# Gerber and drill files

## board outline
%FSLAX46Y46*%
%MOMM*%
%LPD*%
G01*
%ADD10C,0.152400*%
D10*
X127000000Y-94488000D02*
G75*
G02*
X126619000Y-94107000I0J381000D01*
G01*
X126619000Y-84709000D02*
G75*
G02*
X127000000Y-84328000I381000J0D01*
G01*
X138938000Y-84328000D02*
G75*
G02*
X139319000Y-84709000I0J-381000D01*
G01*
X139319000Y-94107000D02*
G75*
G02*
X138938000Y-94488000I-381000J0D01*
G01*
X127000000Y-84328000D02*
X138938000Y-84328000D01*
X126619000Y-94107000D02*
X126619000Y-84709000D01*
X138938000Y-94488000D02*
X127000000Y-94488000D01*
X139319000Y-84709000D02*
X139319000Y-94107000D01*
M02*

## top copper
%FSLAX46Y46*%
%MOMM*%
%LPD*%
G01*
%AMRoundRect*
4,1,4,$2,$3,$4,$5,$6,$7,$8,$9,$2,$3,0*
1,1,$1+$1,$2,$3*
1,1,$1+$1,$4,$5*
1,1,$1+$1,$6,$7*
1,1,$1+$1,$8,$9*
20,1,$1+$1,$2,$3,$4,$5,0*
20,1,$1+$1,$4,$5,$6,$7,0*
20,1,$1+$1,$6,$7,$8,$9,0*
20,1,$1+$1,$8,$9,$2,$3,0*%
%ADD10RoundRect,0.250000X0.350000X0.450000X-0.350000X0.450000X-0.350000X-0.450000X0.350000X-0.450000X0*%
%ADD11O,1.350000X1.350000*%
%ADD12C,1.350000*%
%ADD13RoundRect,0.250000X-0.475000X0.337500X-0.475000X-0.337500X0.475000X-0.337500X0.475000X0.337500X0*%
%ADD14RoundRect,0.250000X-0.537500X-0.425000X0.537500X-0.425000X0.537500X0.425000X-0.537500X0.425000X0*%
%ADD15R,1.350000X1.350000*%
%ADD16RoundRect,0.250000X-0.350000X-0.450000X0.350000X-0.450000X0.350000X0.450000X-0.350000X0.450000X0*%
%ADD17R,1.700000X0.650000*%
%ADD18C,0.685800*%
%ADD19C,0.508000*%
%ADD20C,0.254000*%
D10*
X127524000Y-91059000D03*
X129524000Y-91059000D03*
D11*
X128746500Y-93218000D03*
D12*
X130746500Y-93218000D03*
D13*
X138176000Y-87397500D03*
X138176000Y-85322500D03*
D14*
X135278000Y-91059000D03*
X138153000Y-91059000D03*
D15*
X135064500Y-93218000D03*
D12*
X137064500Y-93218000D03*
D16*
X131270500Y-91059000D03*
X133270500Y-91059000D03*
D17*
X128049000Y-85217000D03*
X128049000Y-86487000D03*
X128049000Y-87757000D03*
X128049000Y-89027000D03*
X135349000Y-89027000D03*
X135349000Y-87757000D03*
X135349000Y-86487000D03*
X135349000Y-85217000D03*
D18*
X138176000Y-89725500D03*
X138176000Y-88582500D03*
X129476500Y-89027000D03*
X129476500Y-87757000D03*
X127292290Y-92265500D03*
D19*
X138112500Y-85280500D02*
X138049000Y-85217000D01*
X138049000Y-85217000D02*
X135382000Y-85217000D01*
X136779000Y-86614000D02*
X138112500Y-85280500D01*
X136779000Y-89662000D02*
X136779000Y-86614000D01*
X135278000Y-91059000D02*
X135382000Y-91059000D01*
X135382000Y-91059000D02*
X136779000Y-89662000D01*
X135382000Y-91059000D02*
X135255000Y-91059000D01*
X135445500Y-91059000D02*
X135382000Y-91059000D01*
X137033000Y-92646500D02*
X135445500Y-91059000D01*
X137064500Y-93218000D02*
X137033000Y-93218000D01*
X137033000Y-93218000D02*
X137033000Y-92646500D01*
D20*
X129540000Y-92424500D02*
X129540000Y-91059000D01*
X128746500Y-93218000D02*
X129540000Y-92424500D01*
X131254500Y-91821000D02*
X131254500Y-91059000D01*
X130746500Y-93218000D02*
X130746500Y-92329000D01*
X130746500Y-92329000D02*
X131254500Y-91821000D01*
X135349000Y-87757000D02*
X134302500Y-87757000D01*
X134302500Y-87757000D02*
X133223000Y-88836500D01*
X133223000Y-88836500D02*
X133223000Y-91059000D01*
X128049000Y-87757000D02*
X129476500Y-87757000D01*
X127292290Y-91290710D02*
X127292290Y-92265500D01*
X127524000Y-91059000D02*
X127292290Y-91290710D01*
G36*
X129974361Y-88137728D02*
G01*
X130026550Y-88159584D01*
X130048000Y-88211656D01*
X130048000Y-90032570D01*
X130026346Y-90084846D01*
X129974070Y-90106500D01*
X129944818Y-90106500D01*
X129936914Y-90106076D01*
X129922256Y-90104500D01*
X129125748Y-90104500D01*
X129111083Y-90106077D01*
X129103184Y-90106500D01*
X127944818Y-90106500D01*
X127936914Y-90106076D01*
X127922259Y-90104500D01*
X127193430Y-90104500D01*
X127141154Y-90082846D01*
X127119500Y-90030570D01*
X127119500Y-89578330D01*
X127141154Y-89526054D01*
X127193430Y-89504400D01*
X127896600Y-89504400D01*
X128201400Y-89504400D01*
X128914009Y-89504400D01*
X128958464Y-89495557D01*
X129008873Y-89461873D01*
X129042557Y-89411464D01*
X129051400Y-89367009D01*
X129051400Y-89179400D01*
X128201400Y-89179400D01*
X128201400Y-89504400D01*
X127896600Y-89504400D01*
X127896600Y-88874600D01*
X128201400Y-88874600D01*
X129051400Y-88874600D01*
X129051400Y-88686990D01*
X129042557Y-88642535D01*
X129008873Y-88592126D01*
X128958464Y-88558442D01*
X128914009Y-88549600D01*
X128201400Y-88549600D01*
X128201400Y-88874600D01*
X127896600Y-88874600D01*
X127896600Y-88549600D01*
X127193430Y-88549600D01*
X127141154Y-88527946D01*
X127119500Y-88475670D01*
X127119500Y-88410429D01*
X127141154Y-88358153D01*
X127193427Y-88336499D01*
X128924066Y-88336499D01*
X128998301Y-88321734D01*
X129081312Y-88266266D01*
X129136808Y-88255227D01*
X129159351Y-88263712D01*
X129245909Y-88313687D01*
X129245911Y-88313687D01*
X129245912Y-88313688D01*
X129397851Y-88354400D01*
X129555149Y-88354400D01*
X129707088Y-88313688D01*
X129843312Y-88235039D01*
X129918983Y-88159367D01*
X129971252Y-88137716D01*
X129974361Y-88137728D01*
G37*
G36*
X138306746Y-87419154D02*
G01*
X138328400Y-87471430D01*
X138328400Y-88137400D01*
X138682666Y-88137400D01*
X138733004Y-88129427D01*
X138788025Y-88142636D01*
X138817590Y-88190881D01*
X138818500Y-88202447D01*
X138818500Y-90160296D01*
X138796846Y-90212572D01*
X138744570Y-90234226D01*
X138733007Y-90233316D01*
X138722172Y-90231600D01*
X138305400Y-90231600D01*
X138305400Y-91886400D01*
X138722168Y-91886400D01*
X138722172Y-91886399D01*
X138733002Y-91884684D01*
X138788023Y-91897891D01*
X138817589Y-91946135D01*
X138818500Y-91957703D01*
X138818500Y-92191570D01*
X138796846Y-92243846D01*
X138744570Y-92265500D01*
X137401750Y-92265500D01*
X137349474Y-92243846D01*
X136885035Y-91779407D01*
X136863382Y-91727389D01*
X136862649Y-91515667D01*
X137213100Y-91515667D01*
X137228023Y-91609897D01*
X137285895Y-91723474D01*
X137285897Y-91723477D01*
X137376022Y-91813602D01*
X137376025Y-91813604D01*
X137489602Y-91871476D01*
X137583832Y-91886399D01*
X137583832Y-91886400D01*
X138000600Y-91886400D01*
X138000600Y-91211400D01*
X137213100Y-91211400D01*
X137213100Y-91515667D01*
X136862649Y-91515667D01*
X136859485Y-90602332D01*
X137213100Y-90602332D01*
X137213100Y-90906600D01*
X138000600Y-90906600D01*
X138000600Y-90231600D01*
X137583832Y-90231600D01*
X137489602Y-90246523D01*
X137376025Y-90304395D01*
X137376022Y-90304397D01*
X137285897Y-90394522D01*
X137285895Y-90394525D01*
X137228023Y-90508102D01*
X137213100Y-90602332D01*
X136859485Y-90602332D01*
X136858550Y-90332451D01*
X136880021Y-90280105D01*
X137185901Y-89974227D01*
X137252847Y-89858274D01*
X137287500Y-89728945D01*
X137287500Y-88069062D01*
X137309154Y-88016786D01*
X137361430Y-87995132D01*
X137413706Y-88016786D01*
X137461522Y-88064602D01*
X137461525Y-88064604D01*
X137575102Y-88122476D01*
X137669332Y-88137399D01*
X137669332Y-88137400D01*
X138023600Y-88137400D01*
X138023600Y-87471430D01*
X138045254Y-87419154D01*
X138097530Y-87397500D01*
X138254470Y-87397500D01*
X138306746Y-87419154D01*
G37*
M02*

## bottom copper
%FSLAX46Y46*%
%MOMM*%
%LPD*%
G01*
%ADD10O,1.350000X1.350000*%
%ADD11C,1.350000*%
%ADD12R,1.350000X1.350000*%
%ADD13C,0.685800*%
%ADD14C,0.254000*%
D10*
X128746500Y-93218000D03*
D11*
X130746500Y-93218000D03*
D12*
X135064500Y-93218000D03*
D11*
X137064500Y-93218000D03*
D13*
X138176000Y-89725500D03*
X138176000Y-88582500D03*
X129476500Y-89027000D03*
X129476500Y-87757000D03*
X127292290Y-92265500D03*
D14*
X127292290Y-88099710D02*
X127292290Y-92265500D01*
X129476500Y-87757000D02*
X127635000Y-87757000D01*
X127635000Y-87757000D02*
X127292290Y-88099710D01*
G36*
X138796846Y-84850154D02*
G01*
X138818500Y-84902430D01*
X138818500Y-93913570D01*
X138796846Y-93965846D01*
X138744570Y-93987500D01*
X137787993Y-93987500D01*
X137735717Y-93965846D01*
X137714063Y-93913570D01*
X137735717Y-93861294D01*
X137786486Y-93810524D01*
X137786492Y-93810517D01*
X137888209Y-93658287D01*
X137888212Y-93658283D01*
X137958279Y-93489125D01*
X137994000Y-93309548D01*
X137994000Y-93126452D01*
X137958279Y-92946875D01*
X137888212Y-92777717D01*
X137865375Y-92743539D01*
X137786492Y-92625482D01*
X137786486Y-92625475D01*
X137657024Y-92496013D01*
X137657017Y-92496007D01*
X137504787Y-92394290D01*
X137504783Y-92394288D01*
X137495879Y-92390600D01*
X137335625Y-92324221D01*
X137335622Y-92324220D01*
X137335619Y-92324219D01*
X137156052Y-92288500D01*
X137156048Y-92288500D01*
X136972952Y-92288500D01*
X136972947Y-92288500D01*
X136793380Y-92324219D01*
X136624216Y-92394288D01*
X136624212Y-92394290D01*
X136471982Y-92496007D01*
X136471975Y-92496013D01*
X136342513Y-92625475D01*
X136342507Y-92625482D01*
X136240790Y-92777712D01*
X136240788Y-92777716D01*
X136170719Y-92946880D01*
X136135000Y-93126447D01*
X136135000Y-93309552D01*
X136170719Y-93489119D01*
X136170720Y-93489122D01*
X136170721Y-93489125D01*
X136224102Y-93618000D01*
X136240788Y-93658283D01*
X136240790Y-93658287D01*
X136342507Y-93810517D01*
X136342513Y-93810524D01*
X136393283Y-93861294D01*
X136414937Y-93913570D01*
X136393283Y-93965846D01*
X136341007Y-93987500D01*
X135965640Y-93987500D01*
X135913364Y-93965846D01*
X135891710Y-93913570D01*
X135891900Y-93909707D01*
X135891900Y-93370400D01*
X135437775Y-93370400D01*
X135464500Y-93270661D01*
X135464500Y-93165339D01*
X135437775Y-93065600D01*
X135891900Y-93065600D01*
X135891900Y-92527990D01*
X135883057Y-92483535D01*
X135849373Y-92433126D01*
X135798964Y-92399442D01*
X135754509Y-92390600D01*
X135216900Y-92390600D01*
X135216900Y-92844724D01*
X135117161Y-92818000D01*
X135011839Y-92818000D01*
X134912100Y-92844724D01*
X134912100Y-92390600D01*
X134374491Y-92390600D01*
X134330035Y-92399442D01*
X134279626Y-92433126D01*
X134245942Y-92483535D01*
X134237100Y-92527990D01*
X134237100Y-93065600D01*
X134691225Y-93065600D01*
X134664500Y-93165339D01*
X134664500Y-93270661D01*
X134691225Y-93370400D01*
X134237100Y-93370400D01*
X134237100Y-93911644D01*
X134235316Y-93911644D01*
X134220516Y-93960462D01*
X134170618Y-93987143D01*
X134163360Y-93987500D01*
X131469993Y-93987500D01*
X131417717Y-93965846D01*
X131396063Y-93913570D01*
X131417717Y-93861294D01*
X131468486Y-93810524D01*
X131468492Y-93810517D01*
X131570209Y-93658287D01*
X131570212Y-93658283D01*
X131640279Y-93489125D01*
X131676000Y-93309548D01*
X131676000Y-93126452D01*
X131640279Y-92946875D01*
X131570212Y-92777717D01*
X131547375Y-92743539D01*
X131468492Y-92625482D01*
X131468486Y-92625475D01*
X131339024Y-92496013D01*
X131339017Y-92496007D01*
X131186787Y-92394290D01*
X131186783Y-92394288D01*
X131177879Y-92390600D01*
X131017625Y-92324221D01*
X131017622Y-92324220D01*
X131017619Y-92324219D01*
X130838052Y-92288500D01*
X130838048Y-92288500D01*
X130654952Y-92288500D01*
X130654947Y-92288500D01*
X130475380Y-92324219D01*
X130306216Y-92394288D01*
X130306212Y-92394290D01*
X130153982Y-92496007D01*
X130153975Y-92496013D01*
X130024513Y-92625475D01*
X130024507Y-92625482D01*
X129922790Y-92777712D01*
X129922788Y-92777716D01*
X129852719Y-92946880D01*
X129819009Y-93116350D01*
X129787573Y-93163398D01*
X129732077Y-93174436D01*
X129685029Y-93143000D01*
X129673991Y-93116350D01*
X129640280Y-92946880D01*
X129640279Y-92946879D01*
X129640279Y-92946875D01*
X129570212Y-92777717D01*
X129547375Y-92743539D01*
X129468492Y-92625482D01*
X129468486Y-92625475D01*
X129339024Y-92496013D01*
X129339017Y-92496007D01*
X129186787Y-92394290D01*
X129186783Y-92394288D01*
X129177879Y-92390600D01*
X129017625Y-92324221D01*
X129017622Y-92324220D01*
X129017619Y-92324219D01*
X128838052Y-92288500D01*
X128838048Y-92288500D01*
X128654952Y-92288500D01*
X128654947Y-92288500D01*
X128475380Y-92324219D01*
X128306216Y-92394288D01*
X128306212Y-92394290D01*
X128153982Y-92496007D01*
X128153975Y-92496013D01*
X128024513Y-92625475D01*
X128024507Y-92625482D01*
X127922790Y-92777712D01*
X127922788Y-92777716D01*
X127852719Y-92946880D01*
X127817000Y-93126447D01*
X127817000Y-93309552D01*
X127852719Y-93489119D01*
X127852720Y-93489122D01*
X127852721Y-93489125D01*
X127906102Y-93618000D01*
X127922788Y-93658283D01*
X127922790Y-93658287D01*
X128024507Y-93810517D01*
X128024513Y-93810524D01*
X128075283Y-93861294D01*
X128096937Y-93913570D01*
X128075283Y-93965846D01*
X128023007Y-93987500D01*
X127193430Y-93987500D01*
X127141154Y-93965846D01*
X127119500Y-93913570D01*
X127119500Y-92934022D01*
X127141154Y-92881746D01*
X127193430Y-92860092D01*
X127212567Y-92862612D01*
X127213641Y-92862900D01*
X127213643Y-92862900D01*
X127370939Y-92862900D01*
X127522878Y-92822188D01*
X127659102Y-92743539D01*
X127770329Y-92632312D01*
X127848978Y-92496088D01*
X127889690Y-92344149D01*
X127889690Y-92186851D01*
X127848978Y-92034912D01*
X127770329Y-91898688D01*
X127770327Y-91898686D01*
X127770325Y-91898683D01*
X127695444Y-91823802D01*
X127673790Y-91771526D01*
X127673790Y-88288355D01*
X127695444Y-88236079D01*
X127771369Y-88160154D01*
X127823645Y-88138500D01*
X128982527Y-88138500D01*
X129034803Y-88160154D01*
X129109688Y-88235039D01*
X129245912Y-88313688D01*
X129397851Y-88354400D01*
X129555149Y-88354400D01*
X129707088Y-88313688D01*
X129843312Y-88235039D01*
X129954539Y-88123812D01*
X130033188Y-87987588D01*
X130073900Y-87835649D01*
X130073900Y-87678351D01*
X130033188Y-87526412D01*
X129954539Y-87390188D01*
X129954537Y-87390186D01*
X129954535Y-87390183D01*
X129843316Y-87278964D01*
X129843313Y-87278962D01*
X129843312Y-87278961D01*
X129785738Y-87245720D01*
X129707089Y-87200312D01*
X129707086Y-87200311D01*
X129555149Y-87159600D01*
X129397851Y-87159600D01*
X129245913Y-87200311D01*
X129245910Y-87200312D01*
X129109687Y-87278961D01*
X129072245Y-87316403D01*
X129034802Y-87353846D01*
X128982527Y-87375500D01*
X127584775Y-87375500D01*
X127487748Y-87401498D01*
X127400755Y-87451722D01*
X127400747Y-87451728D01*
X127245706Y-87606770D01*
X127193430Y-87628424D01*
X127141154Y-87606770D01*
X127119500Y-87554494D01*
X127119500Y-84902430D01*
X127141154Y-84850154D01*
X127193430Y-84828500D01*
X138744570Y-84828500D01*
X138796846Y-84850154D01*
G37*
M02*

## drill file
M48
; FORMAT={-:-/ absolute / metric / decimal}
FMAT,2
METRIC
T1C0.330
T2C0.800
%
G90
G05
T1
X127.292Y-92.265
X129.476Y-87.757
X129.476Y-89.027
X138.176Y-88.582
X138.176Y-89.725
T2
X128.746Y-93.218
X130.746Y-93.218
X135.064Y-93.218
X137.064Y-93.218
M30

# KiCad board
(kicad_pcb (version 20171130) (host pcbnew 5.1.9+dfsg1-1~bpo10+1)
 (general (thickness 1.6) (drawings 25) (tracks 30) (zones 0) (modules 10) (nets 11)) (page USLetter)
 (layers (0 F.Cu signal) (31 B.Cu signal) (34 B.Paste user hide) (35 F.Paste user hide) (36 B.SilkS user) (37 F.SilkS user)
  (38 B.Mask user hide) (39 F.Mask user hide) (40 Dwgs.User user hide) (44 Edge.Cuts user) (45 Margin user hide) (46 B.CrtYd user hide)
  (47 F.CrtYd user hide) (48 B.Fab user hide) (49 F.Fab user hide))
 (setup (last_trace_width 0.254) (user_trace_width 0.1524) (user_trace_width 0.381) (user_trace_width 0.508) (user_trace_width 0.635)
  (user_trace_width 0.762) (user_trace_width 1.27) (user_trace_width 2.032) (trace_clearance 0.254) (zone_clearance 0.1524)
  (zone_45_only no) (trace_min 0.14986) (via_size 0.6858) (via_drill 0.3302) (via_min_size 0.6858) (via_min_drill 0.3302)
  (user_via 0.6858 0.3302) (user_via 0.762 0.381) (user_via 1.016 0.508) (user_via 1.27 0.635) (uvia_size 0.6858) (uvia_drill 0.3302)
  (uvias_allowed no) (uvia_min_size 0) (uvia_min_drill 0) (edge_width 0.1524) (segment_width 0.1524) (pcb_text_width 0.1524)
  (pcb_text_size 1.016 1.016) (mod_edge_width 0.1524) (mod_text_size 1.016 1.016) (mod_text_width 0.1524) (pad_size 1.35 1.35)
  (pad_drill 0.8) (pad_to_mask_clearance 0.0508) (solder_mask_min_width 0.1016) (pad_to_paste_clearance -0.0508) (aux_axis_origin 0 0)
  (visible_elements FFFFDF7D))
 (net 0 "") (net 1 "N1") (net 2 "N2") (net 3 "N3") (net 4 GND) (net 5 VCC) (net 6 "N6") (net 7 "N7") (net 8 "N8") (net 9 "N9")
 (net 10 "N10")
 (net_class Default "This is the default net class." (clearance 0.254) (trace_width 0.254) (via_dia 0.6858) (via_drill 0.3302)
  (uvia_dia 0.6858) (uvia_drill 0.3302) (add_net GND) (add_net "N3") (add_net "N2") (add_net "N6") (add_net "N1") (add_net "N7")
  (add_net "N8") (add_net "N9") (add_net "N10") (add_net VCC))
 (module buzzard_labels (layer B.Cu) (at 135.89 91.3765 180)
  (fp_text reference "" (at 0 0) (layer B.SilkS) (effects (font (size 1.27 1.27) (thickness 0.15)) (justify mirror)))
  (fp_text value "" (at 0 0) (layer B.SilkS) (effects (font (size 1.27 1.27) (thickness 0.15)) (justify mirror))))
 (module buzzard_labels (layer B.Cu) (at 129.667 91.3765 180)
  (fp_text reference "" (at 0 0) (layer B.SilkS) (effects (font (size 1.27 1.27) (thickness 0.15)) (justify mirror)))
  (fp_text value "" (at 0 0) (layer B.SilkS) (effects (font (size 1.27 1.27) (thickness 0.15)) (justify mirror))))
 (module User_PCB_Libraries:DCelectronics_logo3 (layer B.Cu) (at 133.223 86.36 180)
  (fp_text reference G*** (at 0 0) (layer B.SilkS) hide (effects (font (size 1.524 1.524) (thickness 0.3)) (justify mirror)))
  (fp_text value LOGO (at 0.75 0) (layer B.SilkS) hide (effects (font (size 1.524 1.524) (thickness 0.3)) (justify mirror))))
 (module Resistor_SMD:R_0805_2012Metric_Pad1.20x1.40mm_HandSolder (layer F.Cu) (at 128.524 91.059 180)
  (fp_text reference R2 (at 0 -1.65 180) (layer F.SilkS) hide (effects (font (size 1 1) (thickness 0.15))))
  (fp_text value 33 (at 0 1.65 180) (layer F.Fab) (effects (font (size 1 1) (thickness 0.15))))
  (pad 2 smd roundrect (at 1 0 180) (size 1.2 1.4) (layers F.Cu F.Paste F.Mask) (roundrect_rratio 0.208333) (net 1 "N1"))
  (pad 1 smd roundrect (at -1 0 180) (size 1.2 1.4) (layers F.Cu F.Paste F.Mask) (roundrect_rratio 0.208333) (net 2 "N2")))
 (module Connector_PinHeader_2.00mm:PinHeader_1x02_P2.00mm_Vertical (layer F.Cu) (at 130.7465 93.218 270)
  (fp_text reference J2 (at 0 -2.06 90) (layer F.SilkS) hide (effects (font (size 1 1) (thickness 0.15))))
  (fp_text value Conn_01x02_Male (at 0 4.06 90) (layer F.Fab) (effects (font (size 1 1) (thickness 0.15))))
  (pad 2 thru_hole oval (at 0 2 270) (size 1.35 1.35) (drill 0.8) (layers *.Cu *.Mask) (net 2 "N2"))
  (pad 1 thru_hole circle (at 0 0 270) (size 1.35 1.35) (drill 0.8) (layers *.Cu *.Mask) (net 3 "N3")))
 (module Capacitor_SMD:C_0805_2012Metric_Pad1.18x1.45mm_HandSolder (layer F.Cu) (at 138.176 86.36 270)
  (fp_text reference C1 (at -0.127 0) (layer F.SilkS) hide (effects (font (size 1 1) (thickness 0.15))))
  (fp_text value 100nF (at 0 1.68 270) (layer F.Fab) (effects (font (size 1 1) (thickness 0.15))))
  (pad 2 smd roundrect (at 1.0375 0 270) (size 1.175 1.45) (layers F.Cu F.Paste F.Mask) (roundrect_rratio 0.212766) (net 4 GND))
  (pad 1 smd roundrect (at -1.0375 0 270) (size 1.175 1.45) (layers F.Cu F.Paste F.Mask) (roundrect_rratio 0.212766) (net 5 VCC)))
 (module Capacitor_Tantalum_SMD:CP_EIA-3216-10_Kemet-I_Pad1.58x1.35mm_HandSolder (layer F.Cu) (at 136.7155 91.059)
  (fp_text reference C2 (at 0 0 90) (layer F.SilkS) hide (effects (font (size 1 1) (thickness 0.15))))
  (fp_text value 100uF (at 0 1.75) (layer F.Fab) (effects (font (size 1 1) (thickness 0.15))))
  (pad 1 smd roundrect (at -1.4375 0) (size 1.575 1.35) (layers F.Cu F.Paste F.Mask) (roundrect_rratio 0.185185) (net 5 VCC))
  (pad 2 smd roundrect (at 1.4375 0) (size 1.575 1.35) (layers F.Cu F.Paste F.Mask) (roundrect_rratio 0.185185) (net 4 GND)))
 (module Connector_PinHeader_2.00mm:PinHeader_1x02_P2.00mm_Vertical (layer F.Cu) (at 137.0645 93.218 270)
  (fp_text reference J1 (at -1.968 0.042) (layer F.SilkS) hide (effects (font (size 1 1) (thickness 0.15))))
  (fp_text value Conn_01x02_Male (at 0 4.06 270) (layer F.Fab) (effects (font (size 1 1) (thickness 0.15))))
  (pad 2 thru_hole rect (at 0 2 270) (size 1.35 1.35) (drill 0.8) (layers *.Cu *.Mask) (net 4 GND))
  (pad 1 thru_hole circle (at 0 0 270) (size 1.35 1.35) (drill 0.8) (layers *.Cu *.Mask) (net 5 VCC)))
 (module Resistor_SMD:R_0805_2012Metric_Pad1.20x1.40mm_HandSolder (layer F.Cu) (at 132.2705 91.059)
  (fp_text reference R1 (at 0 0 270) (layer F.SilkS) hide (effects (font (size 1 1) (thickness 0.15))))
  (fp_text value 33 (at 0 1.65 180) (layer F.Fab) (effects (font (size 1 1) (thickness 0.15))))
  (pad 1 smd roundrect (at -1 0) (size 1.2 1.4) (layers F.Cu F.Paste F.Mask) (roundrect_rratio 0.208333) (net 3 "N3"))
  (pad 2 smd roundrect (at 1 0) (size 1.2 1.4) (layers F.Cu F.Paste F.Mask) (roundrect_rratio 0.208333) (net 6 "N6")))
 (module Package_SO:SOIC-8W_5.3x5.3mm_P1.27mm (layer F.Cu) (at 131.699 87.122)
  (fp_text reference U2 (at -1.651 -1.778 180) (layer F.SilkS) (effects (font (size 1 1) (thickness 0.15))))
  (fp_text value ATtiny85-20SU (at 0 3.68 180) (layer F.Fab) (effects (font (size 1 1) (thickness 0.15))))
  (pad 1 smd rect (at -3.65 -1.905) (size 1.7 0.65) (layers F.Cu F.Paste F.Mask) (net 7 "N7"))
  (pad 2 smd rect (at -3.65 -0.635) (size 1.7 0.65) (layers F.Cu F.Paste F.Mask) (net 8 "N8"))
  (pad 3 smd rect (at -3.65 0.635) (size 1.7 0.65) (layers F.Cu F.Paste F.Mask) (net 1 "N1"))
  (pad 4 smd rect (at -3.65 1.905) (size 1.7 0.65) (layers F.Cu F.Paste F.Mask) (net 4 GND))
  (pad 5 smd rect (at 3.65 1.905) (size 1.7 0.65) (layers F.Cu F.Paste F.Mask) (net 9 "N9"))
  (pad 6 smd rect (at 3.65 0.635) (size 1.7 0.65) (layers F.Cu F.Paste F.Mask) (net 6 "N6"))
  (pad 7 smd rect (at 3.65 -0.635) (size 1.7 0.65) (layers F.Cu F.Paste F.Mask) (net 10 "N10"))
  (pad 8 smd rect (at 3.65 -1.905) (size 1.7 0.65) (layers F.Cu F.Paste F.Mask) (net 5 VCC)))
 (gr_arc (start 127 94.107) (end 126.619 94.107) (angle -90) (layer Edge.Cuts) (width 0.1524))
 (gr_arc (start 127 84.709) (end 127 84.328) (angle -90) (layer Edge.Cuts) (width 0.1524))
 (gr_arc (start 138.938 84.709) (end 139.319 84.709) (angle -90) (layer Edge.Cuts) (width 0.1524))
 (gr_arc (start 138.938 94.107) (end 138.938 94.488) (angle -90) (layer Edge.Cuts) (width 0.1524))
 (gr_line (start 127 84.328) (end 138.938 84.328) (layer Edge.Cuts) (width 0.1524))
 (gr_line (start 126.619 94.107) (end 126.619 84.709) (layer Edge.Cuts) (width 0.1524))
 (gr_line (start 138.938 94.488) (end 127 94.488) (layer Edge.Cuts) (width 0.1524))
 (gr_line (start 139.319 84.709) (end 139.319 94.107) (layer Edge.Cuts) (width 0.1524))
 (via (at 138.176 89.7255) (size 0.6858) (drill 0.3302) (layers F.Cu B.Cu) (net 4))
 (via (at 138.176 88.5825) (size 0.6858) (drill 0.3302) (layers F.Cu B.Cu) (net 4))
 (via (at 129.4765 89.027) (size 0.6858) (drill 0.3302) (layers F.Cu B.Cu) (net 4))
 (segment (start 138.1125 85.2805) (end 138.049 85.217) (width 0.508) (layer F.Cu) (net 5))
 (segment (start 138.049 85.217) (end 135.382 85.217) (width 0.508) (layer F.Cu) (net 5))
 (segment (start 136.779 86.614) (end 138.1125 85.2805) (width 0.508) (layer F.Cu) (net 5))
 (segment (start 136.779 89.662) (end 136.779 86.614) (width 0.508) (layer F.Cu) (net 5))
 (segment (start 135.278 91.059) (end 135.382 91.059) (width 0.508) (layer F.Cu) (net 5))
 (segment (start 135.382 91.059) (end 136.779 89.662) (width 0.508) (layer F.Cu) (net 5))
 (segment (start 135.382 91.059) (end 135.255 91.059) (width 0.508) (layer F.Cu) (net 5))
 (segment (start 135.4455 91.059) (end 135.382 91.059) (width 0.508) (layer F.Cu) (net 5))
 (segment (start 137.033 92.6465) (end 135.4455 91.059) (width 0.508) (layer F.Cu) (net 5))
 (segment (start 137.0645 93.218) (end 137.033 93.218) (width 0.508) (layer F.Cu) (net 5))
 (segment (start 137.033 93.218) (end 137.033 92.6465) (width 0.508) (layer F.Cu) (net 5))
 (segment (start 129.54 92.4245) (end 129.54 91.059) (width 0.254) (layer F.Cu) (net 2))
 (segment (start 128.7465 93.218) (end 129.54 92.4245) (width 0.254) (layer F.Cu) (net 2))
 (segment (start 131.2545 91.821) (end 131.2545 91.059) (width 0.254) (layer F.Cu) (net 3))
 (segment (start 130.7465 93.218) (end 130.7465 92.329) (width 0.254) (layer F.Cu) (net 3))
 (segment (start 130.7465 92.329) (end 131.2545 91.821) (width 0.254) (layer F.Cu) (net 3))
 (segment (start 135.349 87.757) (end 134.3025 87.757) (width 0.254) (layer F.Cu) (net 6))
 (segment (start 134.3025 87.757) (end 133.223 88.8365) (width 0.254) (layer F.Cu) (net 6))
 (segment (start 133.223 88.8365) (end 133.223 91.059) (width 0.254) (layer F.Cu) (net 6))
 (via (at 129.4765 87.757) (size 0.6858) (drill 0.3302) (layers F.Cu B.Cu) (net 1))
 (segment (start 128.049 87.757) (end 129.4765 87.757) (width 0.254) (layer F.Cu) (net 1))
 (via (at 127.29229 92.2655) (size 0.6858) (drill 0.3302) (layers F.Cu B.Cu) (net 1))
 (segment (start 127.29229 91.29071) (end 127.29229 92.2655) (width 0.254) (layer F.Cu) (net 1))
 (segment (start 127.524 91.059) (end 127.29229 91.29071) (width 0.254) (layer F.Cu) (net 1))
 (segment (start 127.29229 88.09971) (end 127.29229 92.2655) (width 0.254) (layer B.Cu) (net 1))
 (segment (start 129.4765 87.757) (end 127.635 87.757) (width 0.254) (layer B.Cu) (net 1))
 (segment (start 127.635 87.757) (end 127.29229 88.09971) (width 0.254) (layer B.Cu) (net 1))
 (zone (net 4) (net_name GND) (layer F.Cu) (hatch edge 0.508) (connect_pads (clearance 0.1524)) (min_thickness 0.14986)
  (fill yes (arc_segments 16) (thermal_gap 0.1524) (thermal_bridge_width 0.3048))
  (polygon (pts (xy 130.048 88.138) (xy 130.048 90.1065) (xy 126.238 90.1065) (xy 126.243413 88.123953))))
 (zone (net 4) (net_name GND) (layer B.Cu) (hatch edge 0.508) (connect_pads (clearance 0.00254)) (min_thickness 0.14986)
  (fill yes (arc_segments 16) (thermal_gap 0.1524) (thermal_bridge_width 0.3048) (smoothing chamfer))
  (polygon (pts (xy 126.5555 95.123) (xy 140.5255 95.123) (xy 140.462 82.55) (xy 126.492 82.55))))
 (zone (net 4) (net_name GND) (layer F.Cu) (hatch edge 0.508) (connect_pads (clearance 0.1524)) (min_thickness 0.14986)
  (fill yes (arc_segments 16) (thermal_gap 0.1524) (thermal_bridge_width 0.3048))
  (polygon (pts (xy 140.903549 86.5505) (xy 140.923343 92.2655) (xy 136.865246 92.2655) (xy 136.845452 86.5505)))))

